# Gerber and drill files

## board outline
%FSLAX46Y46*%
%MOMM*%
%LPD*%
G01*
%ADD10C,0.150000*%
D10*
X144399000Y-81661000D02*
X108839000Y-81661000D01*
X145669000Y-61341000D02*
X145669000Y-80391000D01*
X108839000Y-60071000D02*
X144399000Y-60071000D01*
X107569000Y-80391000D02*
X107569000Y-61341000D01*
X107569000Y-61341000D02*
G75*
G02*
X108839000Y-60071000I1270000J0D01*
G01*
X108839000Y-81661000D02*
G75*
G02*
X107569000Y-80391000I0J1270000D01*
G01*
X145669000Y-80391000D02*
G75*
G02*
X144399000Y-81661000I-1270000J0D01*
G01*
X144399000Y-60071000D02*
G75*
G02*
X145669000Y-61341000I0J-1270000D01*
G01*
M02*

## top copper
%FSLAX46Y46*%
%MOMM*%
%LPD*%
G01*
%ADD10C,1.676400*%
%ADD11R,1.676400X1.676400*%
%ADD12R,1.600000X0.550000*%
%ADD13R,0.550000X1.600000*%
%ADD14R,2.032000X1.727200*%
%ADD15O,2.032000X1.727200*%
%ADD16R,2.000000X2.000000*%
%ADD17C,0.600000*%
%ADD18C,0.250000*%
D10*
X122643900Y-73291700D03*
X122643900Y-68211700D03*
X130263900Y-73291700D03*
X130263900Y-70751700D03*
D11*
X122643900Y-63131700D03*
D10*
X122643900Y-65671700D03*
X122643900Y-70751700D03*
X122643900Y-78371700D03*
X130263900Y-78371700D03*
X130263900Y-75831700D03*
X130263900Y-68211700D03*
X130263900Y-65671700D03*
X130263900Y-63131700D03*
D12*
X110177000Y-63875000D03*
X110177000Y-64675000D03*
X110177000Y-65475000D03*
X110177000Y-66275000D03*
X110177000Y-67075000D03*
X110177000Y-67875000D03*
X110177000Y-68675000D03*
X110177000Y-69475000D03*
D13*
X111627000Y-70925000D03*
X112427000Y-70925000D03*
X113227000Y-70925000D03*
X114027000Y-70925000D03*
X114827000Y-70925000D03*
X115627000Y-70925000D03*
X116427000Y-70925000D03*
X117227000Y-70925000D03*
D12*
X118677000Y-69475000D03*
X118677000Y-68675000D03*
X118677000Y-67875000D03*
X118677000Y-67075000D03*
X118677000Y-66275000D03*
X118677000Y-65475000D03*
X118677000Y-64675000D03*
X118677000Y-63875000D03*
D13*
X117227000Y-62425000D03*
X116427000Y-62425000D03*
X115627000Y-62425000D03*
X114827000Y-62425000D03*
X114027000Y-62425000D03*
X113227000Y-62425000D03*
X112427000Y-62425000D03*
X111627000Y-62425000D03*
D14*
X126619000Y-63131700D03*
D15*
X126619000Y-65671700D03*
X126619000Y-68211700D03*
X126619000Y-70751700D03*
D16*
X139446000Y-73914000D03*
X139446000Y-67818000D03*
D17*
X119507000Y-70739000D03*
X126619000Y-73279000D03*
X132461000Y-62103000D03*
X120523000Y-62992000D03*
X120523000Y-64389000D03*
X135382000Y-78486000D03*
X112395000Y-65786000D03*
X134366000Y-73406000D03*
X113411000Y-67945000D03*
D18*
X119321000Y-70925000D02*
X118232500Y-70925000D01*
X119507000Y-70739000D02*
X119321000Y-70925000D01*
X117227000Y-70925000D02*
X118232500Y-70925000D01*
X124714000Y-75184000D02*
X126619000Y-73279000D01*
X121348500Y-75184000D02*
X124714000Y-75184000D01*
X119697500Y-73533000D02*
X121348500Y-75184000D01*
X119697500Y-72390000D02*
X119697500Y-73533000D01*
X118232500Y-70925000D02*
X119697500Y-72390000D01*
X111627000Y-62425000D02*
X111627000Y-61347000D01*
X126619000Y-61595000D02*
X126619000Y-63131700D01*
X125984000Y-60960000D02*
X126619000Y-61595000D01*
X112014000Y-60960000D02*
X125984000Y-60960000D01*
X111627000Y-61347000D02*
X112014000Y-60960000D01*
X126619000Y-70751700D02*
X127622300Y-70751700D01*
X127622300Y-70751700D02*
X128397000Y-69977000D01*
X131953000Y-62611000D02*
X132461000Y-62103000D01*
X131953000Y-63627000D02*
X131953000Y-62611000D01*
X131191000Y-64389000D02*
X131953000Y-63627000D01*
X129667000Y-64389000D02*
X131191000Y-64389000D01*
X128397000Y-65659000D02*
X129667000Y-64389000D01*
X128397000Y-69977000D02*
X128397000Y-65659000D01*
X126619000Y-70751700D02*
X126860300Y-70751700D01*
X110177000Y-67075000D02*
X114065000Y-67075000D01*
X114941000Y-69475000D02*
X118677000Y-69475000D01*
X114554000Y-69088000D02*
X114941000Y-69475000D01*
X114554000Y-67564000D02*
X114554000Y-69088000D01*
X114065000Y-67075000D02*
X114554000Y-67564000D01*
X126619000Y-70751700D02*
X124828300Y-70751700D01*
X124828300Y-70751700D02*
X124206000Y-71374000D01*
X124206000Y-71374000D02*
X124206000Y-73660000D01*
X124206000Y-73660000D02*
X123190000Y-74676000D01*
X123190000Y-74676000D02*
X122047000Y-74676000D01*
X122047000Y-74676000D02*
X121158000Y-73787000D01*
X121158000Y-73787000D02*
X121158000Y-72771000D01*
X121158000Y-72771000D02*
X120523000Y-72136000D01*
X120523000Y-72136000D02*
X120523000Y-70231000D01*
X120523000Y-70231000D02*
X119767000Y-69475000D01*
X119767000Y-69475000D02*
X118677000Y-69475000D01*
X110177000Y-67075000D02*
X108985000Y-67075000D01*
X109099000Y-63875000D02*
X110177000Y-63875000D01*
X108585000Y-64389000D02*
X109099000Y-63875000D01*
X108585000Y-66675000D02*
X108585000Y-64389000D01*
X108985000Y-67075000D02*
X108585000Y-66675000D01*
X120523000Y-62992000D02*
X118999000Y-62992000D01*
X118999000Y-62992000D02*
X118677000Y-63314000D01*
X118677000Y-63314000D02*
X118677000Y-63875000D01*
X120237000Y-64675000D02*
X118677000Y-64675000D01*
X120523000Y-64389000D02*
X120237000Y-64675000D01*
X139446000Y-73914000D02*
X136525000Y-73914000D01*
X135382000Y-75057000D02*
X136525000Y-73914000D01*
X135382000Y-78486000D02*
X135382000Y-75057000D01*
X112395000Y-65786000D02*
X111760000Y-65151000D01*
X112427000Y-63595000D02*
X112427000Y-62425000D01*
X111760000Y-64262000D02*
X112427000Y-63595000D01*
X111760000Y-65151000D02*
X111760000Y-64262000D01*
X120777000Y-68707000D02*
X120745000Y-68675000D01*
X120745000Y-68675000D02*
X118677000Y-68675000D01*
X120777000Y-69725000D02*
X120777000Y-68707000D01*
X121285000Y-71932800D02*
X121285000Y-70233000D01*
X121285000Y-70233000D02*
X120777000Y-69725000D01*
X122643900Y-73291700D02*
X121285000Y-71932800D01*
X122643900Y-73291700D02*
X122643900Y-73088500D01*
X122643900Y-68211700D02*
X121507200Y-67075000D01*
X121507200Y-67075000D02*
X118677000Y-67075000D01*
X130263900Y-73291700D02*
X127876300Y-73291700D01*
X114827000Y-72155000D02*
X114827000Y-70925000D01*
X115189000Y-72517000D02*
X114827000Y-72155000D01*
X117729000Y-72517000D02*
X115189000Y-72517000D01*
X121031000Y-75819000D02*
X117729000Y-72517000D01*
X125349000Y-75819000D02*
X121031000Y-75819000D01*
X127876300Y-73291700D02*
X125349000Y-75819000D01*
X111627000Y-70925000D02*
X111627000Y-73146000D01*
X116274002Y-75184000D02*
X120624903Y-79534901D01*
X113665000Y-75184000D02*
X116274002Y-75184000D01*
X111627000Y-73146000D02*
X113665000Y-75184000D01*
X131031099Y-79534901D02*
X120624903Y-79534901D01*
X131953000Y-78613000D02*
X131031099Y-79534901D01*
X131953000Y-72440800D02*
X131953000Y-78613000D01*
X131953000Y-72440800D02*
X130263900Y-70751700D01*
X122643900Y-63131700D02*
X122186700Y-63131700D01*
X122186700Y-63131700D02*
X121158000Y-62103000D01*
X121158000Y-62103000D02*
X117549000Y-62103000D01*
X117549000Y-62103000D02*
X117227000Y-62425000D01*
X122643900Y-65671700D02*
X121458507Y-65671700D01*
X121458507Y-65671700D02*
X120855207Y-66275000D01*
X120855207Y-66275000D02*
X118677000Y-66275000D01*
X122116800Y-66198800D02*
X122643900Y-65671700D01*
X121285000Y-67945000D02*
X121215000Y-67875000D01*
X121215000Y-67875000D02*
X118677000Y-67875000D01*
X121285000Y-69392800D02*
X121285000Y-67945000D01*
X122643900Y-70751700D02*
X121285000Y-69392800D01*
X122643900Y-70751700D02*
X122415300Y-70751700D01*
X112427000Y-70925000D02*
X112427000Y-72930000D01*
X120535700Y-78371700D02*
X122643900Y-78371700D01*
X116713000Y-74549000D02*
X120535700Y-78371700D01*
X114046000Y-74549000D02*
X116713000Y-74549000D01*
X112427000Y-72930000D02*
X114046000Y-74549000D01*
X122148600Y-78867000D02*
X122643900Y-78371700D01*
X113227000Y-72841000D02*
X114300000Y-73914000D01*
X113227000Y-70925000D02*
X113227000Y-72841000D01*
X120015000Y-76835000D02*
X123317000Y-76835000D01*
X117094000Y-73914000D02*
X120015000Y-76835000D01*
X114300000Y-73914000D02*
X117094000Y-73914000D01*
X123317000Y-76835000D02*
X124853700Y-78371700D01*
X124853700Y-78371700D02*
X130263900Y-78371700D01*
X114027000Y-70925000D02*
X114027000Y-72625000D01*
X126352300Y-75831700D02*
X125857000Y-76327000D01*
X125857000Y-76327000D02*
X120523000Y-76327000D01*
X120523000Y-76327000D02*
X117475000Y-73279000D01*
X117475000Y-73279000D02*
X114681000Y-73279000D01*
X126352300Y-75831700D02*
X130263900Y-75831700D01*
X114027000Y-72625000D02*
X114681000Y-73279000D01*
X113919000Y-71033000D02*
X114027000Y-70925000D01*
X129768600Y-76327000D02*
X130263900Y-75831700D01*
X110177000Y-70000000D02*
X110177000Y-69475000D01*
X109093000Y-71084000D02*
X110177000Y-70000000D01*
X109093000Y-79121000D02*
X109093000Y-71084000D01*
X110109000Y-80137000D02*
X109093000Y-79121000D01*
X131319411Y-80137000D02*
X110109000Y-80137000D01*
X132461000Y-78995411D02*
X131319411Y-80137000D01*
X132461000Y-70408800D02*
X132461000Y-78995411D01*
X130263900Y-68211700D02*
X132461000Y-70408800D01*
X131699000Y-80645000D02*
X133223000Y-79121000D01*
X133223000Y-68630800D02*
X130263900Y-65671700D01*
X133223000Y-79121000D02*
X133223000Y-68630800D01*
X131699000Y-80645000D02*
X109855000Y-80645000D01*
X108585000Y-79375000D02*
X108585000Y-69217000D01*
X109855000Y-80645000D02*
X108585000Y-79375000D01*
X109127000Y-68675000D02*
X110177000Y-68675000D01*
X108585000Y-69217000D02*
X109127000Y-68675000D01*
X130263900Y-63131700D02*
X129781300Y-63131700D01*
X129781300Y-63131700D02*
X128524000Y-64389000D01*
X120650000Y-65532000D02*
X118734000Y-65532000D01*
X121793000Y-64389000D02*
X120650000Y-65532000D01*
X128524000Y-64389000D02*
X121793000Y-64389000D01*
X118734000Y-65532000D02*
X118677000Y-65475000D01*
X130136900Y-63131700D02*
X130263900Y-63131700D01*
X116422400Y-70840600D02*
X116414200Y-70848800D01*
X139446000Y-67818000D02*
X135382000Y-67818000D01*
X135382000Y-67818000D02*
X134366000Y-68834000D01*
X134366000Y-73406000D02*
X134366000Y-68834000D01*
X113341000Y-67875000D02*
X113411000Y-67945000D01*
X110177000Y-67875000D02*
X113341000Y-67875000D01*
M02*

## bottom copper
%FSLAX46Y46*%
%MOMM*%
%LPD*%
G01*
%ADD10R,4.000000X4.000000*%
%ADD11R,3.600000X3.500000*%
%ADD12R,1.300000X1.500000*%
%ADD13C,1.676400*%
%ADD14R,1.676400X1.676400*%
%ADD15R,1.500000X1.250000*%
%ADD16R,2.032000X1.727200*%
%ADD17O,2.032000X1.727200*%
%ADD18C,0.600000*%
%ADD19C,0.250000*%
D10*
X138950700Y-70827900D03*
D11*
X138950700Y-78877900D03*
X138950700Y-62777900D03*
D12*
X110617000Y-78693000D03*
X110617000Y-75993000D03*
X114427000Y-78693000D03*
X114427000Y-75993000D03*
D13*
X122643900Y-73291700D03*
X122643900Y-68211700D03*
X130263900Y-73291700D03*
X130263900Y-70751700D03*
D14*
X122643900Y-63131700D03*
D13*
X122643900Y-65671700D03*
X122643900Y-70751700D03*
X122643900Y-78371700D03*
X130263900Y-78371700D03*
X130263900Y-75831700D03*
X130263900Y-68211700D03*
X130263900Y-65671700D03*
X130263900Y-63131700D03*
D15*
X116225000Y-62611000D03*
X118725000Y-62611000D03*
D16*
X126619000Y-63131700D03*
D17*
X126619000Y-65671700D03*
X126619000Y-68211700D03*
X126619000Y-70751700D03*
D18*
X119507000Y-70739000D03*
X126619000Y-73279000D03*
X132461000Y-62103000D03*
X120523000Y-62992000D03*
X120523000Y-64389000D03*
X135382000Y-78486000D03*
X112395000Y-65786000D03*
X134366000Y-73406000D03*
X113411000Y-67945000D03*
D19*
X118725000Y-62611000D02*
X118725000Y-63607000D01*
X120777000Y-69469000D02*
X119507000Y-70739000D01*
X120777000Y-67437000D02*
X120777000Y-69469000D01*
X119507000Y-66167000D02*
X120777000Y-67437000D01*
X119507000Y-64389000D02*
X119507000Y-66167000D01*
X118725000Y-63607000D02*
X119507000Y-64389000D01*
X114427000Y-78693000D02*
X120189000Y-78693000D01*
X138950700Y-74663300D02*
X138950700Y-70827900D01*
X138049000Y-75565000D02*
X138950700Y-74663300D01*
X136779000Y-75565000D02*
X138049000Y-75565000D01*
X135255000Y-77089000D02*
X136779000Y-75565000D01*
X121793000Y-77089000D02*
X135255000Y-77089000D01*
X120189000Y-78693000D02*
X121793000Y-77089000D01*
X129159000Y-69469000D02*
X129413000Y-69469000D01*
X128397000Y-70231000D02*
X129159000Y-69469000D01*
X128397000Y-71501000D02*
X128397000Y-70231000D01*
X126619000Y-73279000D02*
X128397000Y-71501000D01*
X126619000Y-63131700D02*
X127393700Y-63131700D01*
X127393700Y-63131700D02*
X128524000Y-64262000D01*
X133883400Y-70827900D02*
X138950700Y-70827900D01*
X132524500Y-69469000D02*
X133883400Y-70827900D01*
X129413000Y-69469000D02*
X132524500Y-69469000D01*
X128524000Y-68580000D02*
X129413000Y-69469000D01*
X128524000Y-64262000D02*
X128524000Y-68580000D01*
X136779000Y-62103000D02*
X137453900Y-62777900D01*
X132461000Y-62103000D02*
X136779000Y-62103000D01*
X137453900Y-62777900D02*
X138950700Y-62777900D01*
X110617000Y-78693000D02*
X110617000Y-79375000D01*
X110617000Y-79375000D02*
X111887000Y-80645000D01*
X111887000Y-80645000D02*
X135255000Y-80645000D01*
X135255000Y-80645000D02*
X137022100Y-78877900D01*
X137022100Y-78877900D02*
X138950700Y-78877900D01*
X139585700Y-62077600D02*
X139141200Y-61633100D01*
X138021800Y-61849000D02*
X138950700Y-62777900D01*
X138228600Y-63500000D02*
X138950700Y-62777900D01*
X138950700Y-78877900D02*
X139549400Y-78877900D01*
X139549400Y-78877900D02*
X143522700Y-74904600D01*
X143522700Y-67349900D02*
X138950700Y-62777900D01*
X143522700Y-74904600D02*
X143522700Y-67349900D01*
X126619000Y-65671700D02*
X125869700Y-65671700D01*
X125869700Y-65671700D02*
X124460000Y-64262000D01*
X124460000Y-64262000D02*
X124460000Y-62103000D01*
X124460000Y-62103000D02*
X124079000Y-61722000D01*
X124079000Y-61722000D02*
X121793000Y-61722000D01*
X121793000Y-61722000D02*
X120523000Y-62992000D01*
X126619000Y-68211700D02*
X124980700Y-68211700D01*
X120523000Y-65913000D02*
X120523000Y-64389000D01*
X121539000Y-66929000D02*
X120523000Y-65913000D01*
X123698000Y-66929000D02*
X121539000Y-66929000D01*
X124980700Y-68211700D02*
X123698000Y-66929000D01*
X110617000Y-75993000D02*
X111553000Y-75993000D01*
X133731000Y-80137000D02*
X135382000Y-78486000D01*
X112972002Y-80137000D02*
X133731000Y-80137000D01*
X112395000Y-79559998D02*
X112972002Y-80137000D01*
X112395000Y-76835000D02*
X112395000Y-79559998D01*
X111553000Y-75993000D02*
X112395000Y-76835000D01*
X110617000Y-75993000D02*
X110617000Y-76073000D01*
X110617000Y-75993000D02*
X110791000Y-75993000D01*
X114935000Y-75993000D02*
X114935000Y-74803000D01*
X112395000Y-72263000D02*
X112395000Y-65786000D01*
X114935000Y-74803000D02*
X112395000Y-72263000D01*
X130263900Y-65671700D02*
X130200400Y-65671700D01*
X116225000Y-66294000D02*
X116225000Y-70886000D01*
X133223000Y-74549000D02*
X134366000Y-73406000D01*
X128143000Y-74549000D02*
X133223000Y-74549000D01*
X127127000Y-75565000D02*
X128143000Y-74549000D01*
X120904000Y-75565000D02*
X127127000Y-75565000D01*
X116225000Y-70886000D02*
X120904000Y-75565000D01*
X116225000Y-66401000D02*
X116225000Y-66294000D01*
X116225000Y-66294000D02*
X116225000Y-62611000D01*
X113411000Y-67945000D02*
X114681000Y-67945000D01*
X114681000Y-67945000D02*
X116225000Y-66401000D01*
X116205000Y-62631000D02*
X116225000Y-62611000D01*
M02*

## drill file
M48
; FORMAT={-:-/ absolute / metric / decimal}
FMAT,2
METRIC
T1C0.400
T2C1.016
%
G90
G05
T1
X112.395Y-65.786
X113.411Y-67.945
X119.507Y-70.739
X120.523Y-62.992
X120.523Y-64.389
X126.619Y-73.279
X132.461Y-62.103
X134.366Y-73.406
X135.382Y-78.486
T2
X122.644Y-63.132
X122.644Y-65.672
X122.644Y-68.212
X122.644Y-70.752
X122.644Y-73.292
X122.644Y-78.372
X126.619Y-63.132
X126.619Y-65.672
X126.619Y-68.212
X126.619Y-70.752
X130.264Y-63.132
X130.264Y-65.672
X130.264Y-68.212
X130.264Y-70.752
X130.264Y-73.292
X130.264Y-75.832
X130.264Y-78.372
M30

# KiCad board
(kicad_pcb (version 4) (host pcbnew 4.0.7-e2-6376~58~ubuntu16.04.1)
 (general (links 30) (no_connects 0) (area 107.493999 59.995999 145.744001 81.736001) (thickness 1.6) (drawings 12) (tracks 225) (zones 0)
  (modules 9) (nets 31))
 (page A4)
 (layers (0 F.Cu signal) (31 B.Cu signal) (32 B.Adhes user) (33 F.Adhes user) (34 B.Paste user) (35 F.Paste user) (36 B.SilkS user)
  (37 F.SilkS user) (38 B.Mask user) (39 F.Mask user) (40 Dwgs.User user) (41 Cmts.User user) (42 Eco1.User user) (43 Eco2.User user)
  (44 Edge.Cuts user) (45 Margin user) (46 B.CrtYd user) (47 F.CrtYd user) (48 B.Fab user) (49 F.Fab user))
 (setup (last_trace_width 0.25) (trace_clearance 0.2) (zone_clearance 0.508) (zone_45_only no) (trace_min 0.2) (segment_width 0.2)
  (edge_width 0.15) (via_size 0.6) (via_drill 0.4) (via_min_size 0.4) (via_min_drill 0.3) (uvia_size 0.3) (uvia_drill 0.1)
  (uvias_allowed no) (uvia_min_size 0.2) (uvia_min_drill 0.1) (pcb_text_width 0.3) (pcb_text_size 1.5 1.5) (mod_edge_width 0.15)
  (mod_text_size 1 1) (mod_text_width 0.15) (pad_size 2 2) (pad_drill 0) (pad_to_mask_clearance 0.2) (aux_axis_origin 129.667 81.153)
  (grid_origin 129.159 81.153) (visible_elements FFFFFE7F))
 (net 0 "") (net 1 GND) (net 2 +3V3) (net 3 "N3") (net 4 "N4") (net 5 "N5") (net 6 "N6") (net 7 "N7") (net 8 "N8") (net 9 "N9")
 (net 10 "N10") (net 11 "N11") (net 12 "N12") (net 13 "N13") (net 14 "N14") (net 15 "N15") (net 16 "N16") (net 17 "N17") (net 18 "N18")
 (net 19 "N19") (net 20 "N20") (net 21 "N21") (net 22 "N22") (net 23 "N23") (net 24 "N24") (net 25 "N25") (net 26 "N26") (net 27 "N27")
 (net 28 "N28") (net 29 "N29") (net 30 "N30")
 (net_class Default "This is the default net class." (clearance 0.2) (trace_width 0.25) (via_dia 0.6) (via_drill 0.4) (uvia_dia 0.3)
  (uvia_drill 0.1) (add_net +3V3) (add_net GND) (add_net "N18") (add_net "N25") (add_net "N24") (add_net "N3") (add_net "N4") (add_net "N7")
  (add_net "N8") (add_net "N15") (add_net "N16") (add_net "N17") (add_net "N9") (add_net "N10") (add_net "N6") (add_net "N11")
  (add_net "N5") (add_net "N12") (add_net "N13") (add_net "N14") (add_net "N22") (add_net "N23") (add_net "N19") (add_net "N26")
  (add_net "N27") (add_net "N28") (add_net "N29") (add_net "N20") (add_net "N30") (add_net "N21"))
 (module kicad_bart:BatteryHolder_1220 (layer B.Cu) (at 138.9507 70.8279 270)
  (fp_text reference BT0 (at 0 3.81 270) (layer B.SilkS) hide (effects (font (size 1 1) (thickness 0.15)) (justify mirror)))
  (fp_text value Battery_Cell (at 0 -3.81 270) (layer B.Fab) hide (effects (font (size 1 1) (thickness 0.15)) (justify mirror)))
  (pad 2 smd rect (at 0 0 270) (size 4 4) (layers B.Cu B.Paste B.Mask) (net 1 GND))
  (pad 1 smd rect (at 8.05 0 270) (size 3.5 3.6) (layers B.Cu B.Paste B.Mask) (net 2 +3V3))
  (pad 1 smd rect (at -8.05 0 270) (size 3.5 3.6) (layers B.Cu B.Paste B.Mask) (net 2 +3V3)))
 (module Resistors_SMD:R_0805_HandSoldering (layer B.Cu) (at 110.617 77.343 90)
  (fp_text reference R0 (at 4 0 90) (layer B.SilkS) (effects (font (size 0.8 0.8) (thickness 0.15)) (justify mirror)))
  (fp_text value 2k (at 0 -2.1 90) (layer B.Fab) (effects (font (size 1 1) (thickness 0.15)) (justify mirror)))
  (pad 1 smd rect (at -1.35 0 90) (size 1.5 1.3) (layers B.Cu B.Paste B.Mask) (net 2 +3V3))
  (pad 2 smd rect (at 1.35 0 90) (size 1.5 1.3) (layers B.Cu B.Paste B.Mask) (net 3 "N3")))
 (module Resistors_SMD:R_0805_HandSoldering (layer B.Cu) (at 114.427 77.343 90)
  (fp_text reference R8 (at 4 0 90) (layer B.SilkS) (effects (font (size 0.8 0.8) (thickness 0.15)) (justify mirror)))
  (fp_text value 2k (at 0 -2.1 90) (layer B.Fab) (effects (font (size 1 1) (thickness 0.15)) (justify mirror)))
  (pad 1 smd rect (at -1.35 0 90) (size 1.5 1.3) (layers B.Cu B.Paste B.Mask) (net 1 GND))
  (pad 2 smd rect (at 1.35 0 90) (size 1.5 1.3) (layers B.Cu B.Paste B.Mask) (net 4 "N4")))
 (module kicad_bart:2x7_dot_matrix (layer F.Cu) (at 126.4539 70.7517 270)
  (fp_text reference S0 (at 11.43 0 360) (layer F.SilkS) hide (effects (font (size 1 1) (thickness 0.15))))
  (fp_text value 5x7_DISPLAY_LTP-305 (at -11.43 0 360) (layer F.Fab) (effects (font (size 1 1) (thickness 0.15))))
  (pad 5C thru_hole circle (at 2.54 3.81 270) (size 1.6764 1.6764) (drill 1.016) (layers *.Cu *.Mask F.SilkS) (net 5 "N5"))
  (pad 3 thru_hole circle (at -2.54 3.81 270) (size 1.6764 1.6764) (drill 1.016) (layers *.Cu *.Mask F.SilkS) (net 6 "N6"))
  (pad 10 thru_hole circle (at 2.54 -3.81 270) (size 1.6764 1.6764) (drill 1.016) (layers *.Cu *.Mask F.SilkS) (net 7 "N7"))
  (pad 11 thru_hole circle (at 0 -3.81 270) (size 1.6764 1.6764) (drill 1.016) (layers *.Cu *.Mask F.SilkS) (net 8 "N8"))
  (pad 1C thru_hole rect (at -7.62 3.81 270) (size 1.6764 1.6764) (drill 1.016) (layers *.Cu *.Mask F.SilkS) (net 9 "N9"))
  (pad 2 thru_hole circle (at -5.08 3.81 270) (size 1.6764 1.6764) (drill 1.016) (layers *.Cu *.Mask F.SilkS) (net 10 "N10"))
  (pad 4 thru_hole circle (at 0 3.81 270) (size 1.6764 1.6764) (drill 1.016) (layers *.Cu *.Mask F.SilkS) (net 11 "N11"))
  (pad 7 thru_hole circle (at 7.62 3.81 270) (size 1.6764 1.6764) (drill 1.016) (layers *.Cu *.Mask F.SilkS) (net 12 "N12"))
  (pad 8C thru_hole circle (at 7.62 -3.81 270) (size 1.6764 1.6764) (drill 1.016) (layers *.Cu *.Mask F.SilkS) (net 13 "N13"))
  (pad 9 thru_hole circle (at 5.08 -3.81 270) (size 1.6764 1.6764) (drill 1.016) (layers *.Cu *.Mask F.SilkS) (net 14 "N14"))
  (pad 12 thru_hole circle (at -2.54 -3.81 270) (size 1.6764 1.6764) (drill 1.016) (layers *.Cu *.Mask F.SilkS) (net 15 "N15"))
  (pad 13C thru_hole circle (at -5.08 -3.81 270) (size 1.6764 1.6764) (drill 1.016) (layers *.Cu *.Mask F.SilkS) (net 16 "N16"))
  (pad 14C thru_hole circle (at -7.62 -3.81 270) (size 1.6764 1.6764) (drill 1.016) (layers *.Cu *.Mask F.SilkS) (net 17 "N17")))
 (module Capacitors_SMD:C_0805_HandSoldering (layer B.Cu) (at 117.475 62.611)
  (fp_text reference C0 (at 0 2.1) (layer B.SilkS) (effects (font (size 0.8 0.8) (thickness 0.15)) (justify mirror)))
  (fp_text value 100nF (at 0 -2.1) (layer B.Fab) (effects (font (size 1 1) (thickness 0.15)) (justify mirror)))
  (pad 1 smd rect (at -1.25 0) (size 1.5 1.25) (layers B.Cu B.Paste B.Mask) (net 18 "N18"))
  (pad 2 smd rect (at 1.25 0) (size 1.5 1.25) (layers B.Cu B.Paste B.Mask) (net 1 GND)))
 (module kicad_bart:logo (layer F.Cu) (at 140.843 77.851)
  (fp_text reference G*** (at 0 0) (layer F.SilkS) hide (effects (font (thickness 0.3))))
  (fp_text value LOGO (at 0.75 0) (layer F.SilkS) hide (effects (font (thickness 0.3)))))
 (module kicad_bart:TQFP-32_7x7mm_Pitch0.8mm (layer F.Cu) (at 114.427 66.675)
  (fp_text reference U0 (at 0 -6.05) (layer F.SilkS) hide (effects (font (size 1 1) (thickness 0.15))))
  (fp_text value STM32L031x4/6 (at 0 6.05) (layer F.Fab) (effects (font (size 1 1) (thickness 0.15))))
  (pad 1 smd rect (at -4.25 -2.8) (size 1.6 0.55) (layers F.Cu F.Paste F.Mask) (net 2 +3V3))
  (pad 2 smd rect (at -4.25 -2) (size 1.6 0.55) (layers F.Cu F.Paste F.Mask) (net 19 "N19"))
  (pad 3 smd rect (at -4.25 -1.2) (size 1.6 0.55) (layers F.Cu F.Paste F.Mask) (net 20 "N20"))
  (pad 4 smd rect (at -4.25 -0.4) (size 1.6 0.55) (layers F.Cu F.Paste F.Mask) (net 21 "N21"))
  (pad 5 smd rect (at -4.25 0.4) (size 1.6 0.55) (layers F.Cu F.Paste F.Mask) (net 2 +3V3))
  (pad 6 smd rect (at -4.25 1.2) (size 1.6 0.55) (layers F.Cu F.Paste F.Mask) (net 18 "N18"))
  (pad 7 smd rect (at -4.25 2) (size 1.6 0.55) (layers F.Cu F.Paste F.Mask) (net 16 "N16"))
  (pad 8 smd rect (at -4.25 2.8) (size 1.6 0.55) (layers F.Cu F.Paste F.Mask) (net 15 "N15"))
  (pad 9 smd rect (at -2.8 4.25 90) (size 1.6 0.55) (layers F.Cu F.Paste F.Mask) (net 8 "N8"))
  (pad 10 smd rect (at -2 4.25 90) (size 1.6 0.55) (layers F.Cu F.Paste F.Mask) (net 12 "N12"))
  (pad 11 smd rect (at -1.2 4.25 90) (size 1.6 0.55) (layers F.Cu F.Paste F.Mask) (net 13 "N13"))
  (pad 12 smd rect (at -0.4 4.25 90) (size 1.6 0.55) (layers F.Cu F.Paste F.Mask) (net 14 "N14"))
  (pad 13 smd rect (at 0.4 4.25 90) (size 1.6 0.55) (layers F.Cu F.Paste F.Mask) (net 7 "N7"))
  (pad 14 smd rect (at 1.2 4.25 90) (size 1.6 0.55) (layers F.Cu F.Paste F.Mask) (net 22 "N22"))
  (pad 15 smd rect (at 2 4.25 90) (size 1.6 0.55) (layers F.Cu F.Paste F.Mask) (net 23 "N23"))
  (pad 16 smd rect (at 2.8 4.25 90) (size 1.6 0.55) (layers F.Cu F.Paste F.Mask) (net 1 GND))
  (pad 17 smd rect (at 4.25 2.8) (size 1.6 0.55) (layers F.Cu F.Paste F.Mask) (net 2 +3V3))
  (pad 18 smd rect (at 4.25 2) (size 1.6 0.55) (layers F.Cu F.Paste F.Mask) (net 5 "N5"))
  (pad 19 smd rect (at 4.25 1.2) (size 1.6 0.55) (layers F.Cu F.Paste F.Mask) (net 11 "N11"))
  (pad 20 smd rect (at 4.25 0.4) (size 1.6 0.55) (layers F.Cu F.Paste F.Mask) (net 6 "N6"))
  (pad 21 smd rect (at 4.25 -0.4) (size 1.6 0.55) (layers F.Cu F.Paste F.Mask) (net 10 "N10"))
  (pad 22 smd rect (at 4.25 -1.2) (size 1.6 0.55) (layers F.Cu F.Paste F.Mask) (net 17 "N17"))
  (pad 23 smd rect (at 4.25 -2) (size 1.6 0.55) (layers F.Cu F.Paste F.Mask) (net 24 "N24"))
  (pad 24 smd rect (at 4.25 -2.8) (size 1.6 0.55) (layers F.Cu F.Paste F.Mask) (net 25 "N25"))
  (pad 25 smd rect (at 2.8 -4.25 90) (size 1.6 0.55) (layers F.Cu F.Paste F.Mask) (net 9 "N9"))
  (pad 26 smd rect (at 2 -4.25 90) (size 1.6 0.55) (layers F.Cu F.Paste F.Mask) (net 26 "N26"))
  (pad 27 smd rect (at 1.2 -4.25 90) (size 1.6 0.55) (layers F.Cu F.Paste F.Mask) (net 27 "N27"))
  (pad 28 smd rect (at 0.4 -4.25 90) (size 1.6 0.55) (layers F.Cu F.Paste F.Mask) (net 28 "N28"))
  (pad 29 smd rect (at -0.4 -4.25 90) (size 1.6 0.55) (layers F.Cu F.Paste F.Mask) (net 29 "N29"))
  (pad 30 smd rect (at -1.2 -4.25 90) (size 1.6 0.55) (layers F.Cu F.Paste F.Mask) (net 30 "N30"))
  (pad 31 smd rect (at -2 -4.25 90) (size 1.6 0.55) (layers F.Cu F.Paste F.Mask) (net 4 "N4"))
  (pad 32 smd rect (at -2.8 -4.25 90) (size 1.6 0.55) (layers F.Cu F.Paste F.Mask) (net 1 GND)))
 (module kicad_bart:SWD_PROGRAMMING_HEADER (layer F.Cu) (at 126.619 63.1317)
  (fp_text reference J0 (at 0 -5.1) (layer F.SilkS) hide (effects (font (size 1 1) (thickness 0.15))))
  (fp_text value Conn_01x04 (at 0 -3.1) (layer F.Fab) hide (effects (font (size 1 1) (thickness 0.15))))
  (pad 1 thru_hole rect (at 0 0) (size 2.032 1.7272) (drill 1.016) (layers *.Cu *.Mask F.SilkS) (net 1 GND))
  (pad 2 thru_hole oval (at 0 2.54) (size 2.032 1.7272) (drill 1.016) (layers *.Cu *.Mask F.SilkS) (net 25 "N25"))
  (pad 3 thru_hole oval (at 0 5.08) (size 2.032 1.7272) (drill 1.016) (layers *.Cu *.Mask F.SilkS) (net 24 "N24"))
  (pad 4 thru_hole oval (at 0 7.62) (size 2.032 1.7272) (drill 1.016) (layers *.Cu *.Mask F.SilkS) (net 2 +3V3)))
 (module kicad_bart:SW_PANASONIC (layer F.Cu) (at 139.446 70.866 270)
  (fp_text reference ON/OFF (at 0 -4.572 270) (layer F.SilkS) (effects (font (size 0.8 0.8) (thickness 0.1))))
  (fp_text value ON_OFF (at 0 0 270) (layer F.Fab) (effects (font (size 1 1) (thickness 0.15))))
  (pad 2 smd rect (at 3.048 0 270) (size 2 2) (layers F.Cu F.Paste F.Mask) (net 3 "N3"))
  (pad 1 smd rect (at -3.048 0 270) (size 2 2) (layers F.Cu F.Paste F.Mask) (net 18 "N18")))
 (gr_line (start 144.399 81.661) (end 108.839 81.661) (angle 90) (layer Edge.Cuts) (width 0.15))
 (gr_line (start 145.669 61.341) (end 145.669 80.391) (angle 90) (layer Edge.Cuts) (width 0.15))
 (gr_line (start 108.839 60.071) (end 144.399 60.071) (angle 90) (layer Edge.Cuts) (width 0.15))
 (gr_line (start 107.569 80.391) (end 107.569 61.341) (angle 90) (layer Edge.Cuts) (width 0.15))
 (gr_arc (start 108.839 61.341) (end 107.569 61.341) (angle 90) (layer Edge.Cuts) (width 0.15))
 (gr_arc (start 108.839 80.391) (end 108.839 81.661) (angle 90) (layer Edge.Cuts) (width 0.15))
 (gr_arc (start 144.399 80.391) (end 145.669 80.391) (angle 90) (layer Edge.Cuts) (width 0.15))
 (gr_arc (start 144.399 61.341) (end 144.399 60.071) (angle 90) (layer Edge.Cuts) (width 0.15))
 (segment (start 118.725 62.611) (end 118.725 63.607) (width 0.25) (layer B.Cu) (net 1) (status 10))
 (segment (start 119.321 70.925) (end 118.2325 70.925) (width 0.25) (layer F.Cu) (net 1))
 (segment (start 119.507 70.739) (end 119.321 70.925) (width 0.25) (layer F.Cu) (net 1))
 (via (at 119.507 70.739) (size 0.6) (drill 0.4) (layers F.Cu B.Cu) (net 1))
 (segment (start 120.777 69.469) (end 119.507 70.739) (width 0.25) (layer B.Cu) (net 1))
 (segment (start 120.777 67.437) (end 120.777 69.469) (width 0.25) (layer B.Cu) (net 1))
 (segment (start 119.507 66.167) (end 120.777 67.437) (width 0.25) (layer B.Cu) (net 1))
 (segment (start 119.507 64.389) (end 119.507 66.167) (width 0.25) (layer B.Cu) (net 1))
 (segment (start 118.725 63.607) (end 119.507 64.389) (width 0.25) (layer B.Cu) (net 1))
 (segment (start 114.427 78.693) (end 120.189 78.693) (width 0.25) (layer B.Cu) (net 1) (status 10))
 (segment (start 138.9507 74.6633) (end 138.9507 70.8279) (width 0.25) (layer B.Cu) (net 1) (status 20))
 (segment (start 138.049 75.565) (end 138.9507 74.6633) (width 0.25) (layer B.Cu) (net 1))
 (segment (start 136.779 75.565) (end 138.049 75.565) (width 0.25) (layer B.Cu) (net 1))
 (segment (start 135.255 77.089) (end 136.779 75.565) (width 0.25) (layer B.Cu) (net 1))
 (segment (start 121.793 77.089) (end 135.255 77.089) (width 0.25) (layer B.Cu) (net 1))
 (segment (start 120.189 78.693) (end 121.793 77.089) (width 0.25) (layer B.Cu) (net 1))
 (segment (start 117.227 70.925) (end 118.2325 70.925) (width 0.25) (layer F.Cu) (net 1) (status 10))
 (segment (start 129.159 69.469) (end 129.413 69.469) (width 0.25) (layer B.Cu) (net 1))
 (segment (start 128.397 70.231) (end 129.159 69.469) (width 0.25) (layer B.Cu) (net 1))
 (segment (start 128.397 71.501) (end 128.397 70.231) (width 0.25) (layer B.Cu) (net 1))
 (segment (start 126.619 73.279) (end 128.397 71.501) (width 0.25) (layer B.Cu) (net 1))
 (via (at 126.619 73.279) (size 0.6) (drill 0.4) (layers F.Cu B.Cu) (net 1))
 (segment (start 124.714 75.184) (end 126.619 73.279) (width 0.25) (layer F.Cu) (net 1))
 (segment (start 121.3485 75.184) (end 124.714 75.184) (width 0.25) (layer F.Cu) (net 1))
 (segment (start 119.6975 73.533) (end 121.3485 75.184) (width 0.25) (layer F.Cu) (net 1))
 (segment (start 119.6975 72.39) (end 119.6975 73.533) (width 0.25) (layer F.Cu) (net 1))
 (segment (start 118.2325 70.925) (end 119.6975 72.39) (width 0.25) (layer F.Cu) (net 1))
 (segment (start 126.619 63.1317) (end 127.3937 63.1317) (width 0.25) (layer B.Cu) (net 1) (status 30))
 (segment (start 127.3937 63.1317) (end 128.524 64.262) (width 0.25) (layer B.Cu) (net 1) (status 10))
 (segment (start 133.8834 70.8279) (end 138.9507 70.8279) (width 0.25) (layer B.Cu) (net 1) (status 20))
 (segment (start 132.5245 69.469) (end 133.8834 70.8279) (width 0.25) (layer B.Cu) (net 1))
 (segment (start 129.413 69.469) (end 132.5245 69.469) (width 0.25) (layer B.Cu) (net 1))
 (segment (start 128.524 68.58) (end 129.413 69.469) (width 0.25) (layer B.Cu) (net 1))
 (segment (start 128.524 64.262) (end 128.524 68.58) (width 0.25) (layer B.Cu) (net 1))
 (segment (start 111.627 62.425) (end 111.627 61.347) (width 0.25) (layer F.Cu) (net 1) (status 10))
 (segment (start 126.619 61.595) (end 126.619 63.1317) (width 0.25) (layer F.Cu) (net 1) (status 20))
 (segment (start 125.984 60.96) (end 126.619 61.595) (width 0.25) (layer F.Cu) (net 1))
 (segment (start 112.014 60.96) (end 125.984 60.96) (width 0.25) (layer F.Cu) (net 1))
 (segment (start 111.627 61.347) (end 112.014 60.96) (width 0.25) (layer F.Cu) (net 1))
 (segment (start 126.619 70.7517) (end 127.6223 70.7517) (width 0.25) (layer F.Cu) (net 2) (status 30))
 (segment (start 127.6223 70.7517) (end 128.397 69.977) (width 0.25) (layer F.Cu) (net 2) (status 10))
 (segment (start 136.779 62.103) (end 137.4539 62.7779) (width 0.25) (layer B.Cu) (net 2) (status 20))
 (segment (start 132.461 62.103) (end 136.779 62.103) (width 0.25) (layer B.Cu) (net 2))
 (via (at 132.461 62.103) (size 0.6) (drill 0.4) (layers F.Cu B.Cu) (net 2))
 (segment (start 131.953 62.611) (end 132.461 62.103) (width 0.25) (layer F.Cu) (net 2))
 (segment (start 131.953 63.627) (end 131.953 62.611) (width 0.25) (layer F.Cu) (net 2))
 (segment (start 131.191 64.389) (end 131.953 63.627) (width 0.25) (layer F.Cu) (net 2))
 (segment (start 129.667 64.389) (end 131.191 64.389) (width 0.25) (layer F.Cu) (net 2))
 (segment (start 128.397 65.659) (end 129.667 64.389) (width 0.25) (layer F.Cu) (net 2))
 (segment (start 128.397 69.977) (end 128.397 65.659) (width 0.25) (layer F.Cu) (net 2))
 (segment (start 137.4539 62.7779) (end 138.9507 62.7779) (width 0.25) (layer B.Cu) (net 2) (status 30))
 (segment (start 110.617 78.693) (end 110.617 79.375) (width 0.25) (layer B.Cu) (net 2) (status 30))
 (segment (start 110.617 79.375) (end 111.887 80.645) (width 0.25) (layer B.Cu) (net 2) (status 10))
 (segment (start 111.887 80.645) (end 135.255 80.645) (width 0.25) (layer B.Cu) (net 2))
 (segment (start 135.255 80.645) (end 137.0221 78.8779) (width 0.25) (layer B.Cu) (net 2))
 (segment (start 137.0221 78.8779) (end 138.9507 78.8779) (width 0.25) (layer B.Cu) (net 2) (status 20))
 (segment (start 126.619 70.7517) (end 126.8603 70.7517) (width 0.25) (layer F.Cu) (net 2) (status 30))
 (segment (start 110.177 67.075) (end 114.065 67.075) (width 0.25) (layer F.Cu) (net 2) (status 10))
 (segment (start 114.941 69.475) (end 118.677 69.475) (width 0.25) (layer F.Cu) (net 2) (status 20))
 (segment (start 114.554 69.088) (end 114.941 69.475) (width 0.25) (layer F.Cu) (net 2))
 (segment (start 114.554 67.564) (end 114.554 69.088) (width 0.25) (layer F.Cu) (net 2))
 (segment (start 114.065 67.075) (end 114.554 67.564) (width 0.25) (layer F.Cu) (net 2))
 (segment (start 126.619 70.7517) (end 124.8283 70.7517) (width 0.25) (layer F.Cu) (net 2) (status 10))
 (segment (start 124.8283 70.7517) (end 124.206 71.374) (width 0.25) (layer F.Cu) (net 2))
 (segment (start 124.206 71.374) (end 124.206 73.66) (width 0.25) (layer F.Cu) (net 2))
 (segment (start 124.206 73.66) (end 123.19 74.676) (width 0.25) (layer F.Cu) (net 2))
 (segment (start 123.19 74.676) (end 122.047 74.676) (width 0.25) (layer F.Cu) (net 2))
 (segment (start 122.047 74.676) (end 121.158 73.787) (width 0.25) (layer F.Cu) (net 2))
 (segment (start 121.158 73.787) (end 121.158 72.771) (width 0.25) (layer F.Cu) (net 2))
 (segment (start 121.158 72.771) (end 120.523 72.136) (width 0.25) (layer F.Cu) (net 2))
 (segment (start 120.523 72.136) (end 120.523 70.231) (width 0.25) (layer F.Cu) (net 2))
 (segment (start 120.523 70.231) (end 119.767 69.475) (width 0.25) (layer F.Cu) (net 2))
 (segment (start 119.767 69.475) (end 118.677 69.475) (width 0.25) (layer F.Cu) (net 2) (status 20))
 (segment (start 110.177 67.075) (end 108.985 67.075) (width 0.25) (layer F.Cu) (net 2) (status 10))
 (segment (start 109.099 63.875) (end 110.177 63.875) (width 0.25) (layer F.Cu) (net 2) (status 20))
 (segment (start 108.585 64.389) (end 109.099 63.875) (width 0.25) (layer F.Cu) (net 2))
 (segment (start 108.585 66.675) (end 108.585 64.389) (width 0.25) (layer F.Cu) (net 2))
 (segment (start 108.985 67.075) (end 108.585 66.675) (width 0.25) (layer F.Cu) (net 2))
 (segment (start 139.5857 62.0776) (end 139.1412 61.6331) (width 0.25) (layer B.Cu) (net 2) (status 30))
 (segment (start 138.0218 61.849) (end 138.9507 62.7779) (width 0.25) (layer B.Cu) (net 2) (status 30))
 (segment (start 138.2286 63.5) (end 138.9507 62.7779) (width 0.25) (layer B.Cu) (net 2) (status 30))
 (segment (start 138.9507 78.8779) (end 139.5494 78.8779) (width 0.25) (layer B.Cu) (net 2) (status 30))
 (segment (start 139.5494 78.8779) (end 143.5227 74.9046) (width 0.25) (layer B.Cu) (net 2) (status 10))
 (segment (start 143.5227 67.3499) (end 138.9507 62.7779) (width 0.25) (layer B.Cu) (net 2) (status 20))
 (segment (start 143.5227 74.9046) (end 143.5227 67.3499) (width 0.25) (layer B.Cu) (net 2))
 (segment (start 126.619 65.6717) (end 125.8697 65.6717) (width 0.25) (layer B.Cu) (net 25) (status 30))
 (segment (start 125.8697 65.6717) (end 124.46 64.262) (width 0.25) (layer B.Cu) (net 25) (status 10))
 (segment (start 124.46 64.262) (end 124.46 62.103) (width 0.25) (layer B.Cu) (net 25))
 (segment (start 124.46 62.103) (end 124.079 61.722) (width 0.25) (layer B.Cu) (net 25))
 (segment (start 124.079 61.722) (end 121.793 61.722) (width 0.25) (layer B.Cu) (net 25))
 (segment (start 121.793 61.722) (end 120.523 62.992) (width 0.25) (layer B.Cu) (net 25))
 (via (at 120.523 62.992) (size 0.6) (drill 0.4) (layers F.Cu B.Cu) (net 25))
 (segment (start 120.523 62.992) (end 118.999 62.992) (width 0.25) (layer F.Cu) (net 25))
 (segment (start 118.999 62.992) (end 118.677 63.314) (width 0.25) (layer F.Cu) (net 25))
 (segment (start 118.677 63.314) (end 118.677 63.875) (width 0.25) (layer F.Cu) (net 25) (status 20))
 (segment (start 126.619 68.2117) (end 124.9807 68.2117) (width 0.25) (layer B.Cu) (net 24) (status 10))
 (segment (start 120.237 64.675) (end 118.677 64.675) (width 0.25) (layer F.Cu) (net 24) (status 20))
 (segment (start 120.523 64.389) (end 120.237 64.675) (width 0.25) (layer F.Cu) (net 24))
 (via (at 120.523 64.389) (size 0.6) (drill 0.4) (layers F.Cu B.Cu) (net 24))
 (segment (start 120.523 65.913) (end 120.523 64.389) (width 0.25) (layer B.Cu) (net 24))
 (segment (start 121.539 66.929) (end 120.523 65.913) (width 0.25) (layer B.Cu) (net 24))
 (segment (start 123.698 66.929) (end 121.539 66.929) (width 0.25) (layer B.Cu) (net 24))
 (segment (start 124.9807 68.2117) (end 123.698 66.929) (width 0.25) (layer B.Cu) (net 24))
 (segment (start 139.446 73.914) (end 136.525 73.914) (width 0.25) (layer F.Cu) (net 3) (status 10))
 (segment (start 110.617 75.993) (end 111.553 75.993) (width 0.25) (layer B.Cu) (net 3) (status 10))
 (segment (start 135.382 75.057) (end 136.525 73.914) (width 0.25) (layer F.Cu) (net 3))
 (segment (start 135.382 78.486) (end 135.382 75.057) (width 0.25) (layer F.Cu) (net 3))
 (via (at 135.382 78.486) (size 0.6) (drill 0.4) (layers F.Cu B.Cu) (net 3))
 (segment (start 133.731 80.137) (end 135.382 78.486) (width 0.25) (layer B.Cu) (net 3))
 (segment (start 112.972002 80.137) (end 133.731 80.137) (width 0.25) (layer B.Cu) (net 3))
 (segment (start 112.395 79.559998) (end 112.972002 80.137) (width 0.25) (layer B.Cu) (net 3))
 (segment (start 112.395 76.835) (end 112.395 79.559998) (width 0.25) (layer B.Cu) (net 3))
 (segment (start 111.553 75.993) (end 112.395 76.835) (width 0.25) (layer B.Cu) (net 3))
 (segment (start 110.617 75.993) (end 110.617 76.073) (width 0.25) (layer B.Cu) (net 3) (status 30))
 (segment (start 110.617 75.993) (end 110.791 75.993) (width 0.25) (layer B.Cu) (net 3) (status 30))
 (segment (start 112.395 65.786) (end 111.76 65.151) (width 0.25) (layer F.Cu) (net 4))
 (segment (start 112.427 63.595) (end 112.427 62.425) (width 0.25) (layer F.Cu) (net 4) (status 20))
 (segment (start 111.76 64.262) (end 112.427 63.595) (width 0.25) (layer F.Cu) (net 4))
 (segment (start 111.76 65.151) (end 111.76 64.262) (width 0.25) (layer F.Cu) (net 4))
 (segment (start 114.935 75.993) (end 114.935 74.803) (width 0.25) (layer B.Cu) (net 4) (status 10))
 (via (at 112.395 65.786) (size 0.6) (drill 0.4) (layers F.Cu B.Cu) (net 4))
 (segment (start 112.395 72.263) (end 112.395 65.786) (width 0.25) (layer B.Cu) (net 4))
 (segment (start 114.935 74.803) (end 112.395 72.263) (width 0.25) (layer B.Cu) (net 4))
 (segment (start 120.777 68.707) (end 120.745 68.675) (width 0.25) (layer F.Cu) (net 5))
 (segment (start 120.745 68.675) (end 118.677 68.675) (width 0.25) (layer F.Cu) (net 5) (status 20))
 (segment (start 120.777 69.725) (end 120.777 68.707) (width 0.25) (layer F.Cu) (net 5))
 (segment (start 121.285 71.9328) (end 121.285 70.233) (width 0.25) (layer F.Cu) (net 5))
 (segment (start 121.285 70.233) (end 120.777 69.725) (width 0.25) (layer F.Cu) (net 5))
 (segment (start 122.6439 73.2917) (end 121.285 71.9328) (width 0.25) (layer F.Cu) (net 5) (status 10))
 (segment (start 122.6439 73.2917) (end 122.6439 73.0885) (width 0.25) (layer F.Cu) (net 5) (status 30))
 (segment (start 122.6439 68.2117) (end 121.5072 67.075) (width 0.25) (layer F.Cu) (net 6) (status 10))
 (segment (start 121.5072 67.075) (end 118.677 67.075) (width 0.25) (layer F.Cu) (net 6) (status 20))
 (segment (start 130.2639 73.2917) (end 127.8763 73.2917) (width 0.25) (layer F.Cu) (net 7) (status 10))
 (segment (start 114.827 72.155) (end 114.827 70.925) (width 0.25) (layer F.Cu) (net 7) (status 20))
 (segment (start 115.189 72.517) (end 114.827 72.155) (width 0.25) (layer F.Cu) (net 7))
 (segment (start 117.729 72.517) (end 115.189 72.517) (width 0.25) (layer F.Cu) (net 7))
 (segment (start 121.031 75.819) (end 117.729 72.517) (width 0.25) (layer F.Cu) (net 7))
 (segment (start 125.349 75.819) (end 121.031 75.819) (width 0.25) (layer F.Cu) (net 7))
 (segment (start 127.8763 73.2917) (end 125.349 75.819) (width 0.25) (layer F.Cu) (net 7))
 (segment (start 111.627 70.925) (end 111.627 73.146) (width 0.25) (layer F.Cu) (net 8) (status 10))
 (segment (start 116.274002 75.184) (end 120.624903 79.534901) (width 0.25) (layer F.Cu) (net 8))
 (segment (start 113.665 75.184) (end 116.274002 75.184) (width 0.25) (layer F.Cu) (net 8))
 (segment (start 111.627 73.146) (end 113.665 75.184) (width 0.25) (layer F.Cu) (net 8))
 (segment (start 131.031099 79.534901) (end 120.624903 79.534901) (width 0.25) (layer F.Cu) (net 8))
 (segment (start 131.953 78.613) (end 131.031099 79.534901) (width 0.25) (layer F.Cu) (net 8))
 (segment (start 131.953 72.4408) (end 131.953 78.613) (width 0.25) (layer F.Cu) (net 8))
 (segment (start 131.953 72.4408) (end 130.2639 70.7517) (width 0.25) (layer F.Cu) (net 8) (status 20))
 (segment (start 122.6439 63.1317) (end 122.1867 63.1317) (width 0.25) (layer F.Cu) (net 9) (status 30))
 (segment (start 122.1867 63.1317) (end 121.158 62.103) (width 0.25) (layer F.Cu) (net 9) (status 10))
 (segment (start 121.158 62.103) (end 117.549 62.103) (width 0.25) (layer F.Cu) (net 9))
 (segment (start 117.549 62.103) (end 117.227 62.425) (width 0.25) (layer F.Cu) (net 9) (status 20))
 (segment (start 122.6439 65.6717) (end 121.458507 65.6717) (width 0.25) (layer F.Cu) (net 10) (status 10))
 (segment (start 121.458507 65.6717) (end 120.855207 66.275) (width 0.25) (layer F.Cu) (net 10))
 (segment (start 120.855207 66.275) (end 118.677 66.275) (width 0.25) (layer F.Cu) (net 10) (status 20))
 (segment (start 122.1168 66.1988) (end 122.6439 65.6717) (width 0.25) (layer F.Cu) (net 10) (status 30))
 (segment (start 121.285 67.945) (end 121.215 67.875) (width 0.25) (layer F.Cu) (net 11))
 (segment (start 121.215 67.875) (end 118.677 67.875) (width 0.25) (layer F.Cu) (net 11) (status 20))
 (segment (start 121.285 69.3928) (end 121.285 67.945) (width 0.25) (layer F.Cu) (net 11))
 (segment (start 122.6439 70.7517) (end 121.285 69.3928) (width 0.25) (layer F.Cu) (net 11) (status 10))
 (segment (start 122.6439 70.7517) (end 122.4153 70.7517) (width 0.25) (layer F.Cu) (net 11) (status 30))
 (segment (start 112.427 70.925) (end 112.427 72.93) (width 0.25) (layer F.Cu) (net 12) (status 10))
 (segment (start 120.5357 78.3717) (end 122.6439 78.3717) (width 0.25) (layer F.Cu) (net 12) (status 20))
 (segment (start 116.713 74.549) (end 120.5357 78.3717) (width 0.25) (layer F.Cu) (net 12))
 (segment (start 114.046 74.549) (end 116.713 74.549) (width 0.25) (layer F.Cu) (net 12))
 (segment (start 112.427 72.93) (end 114.046 74.549) (width 0.25) (layer F.Cu) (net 12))
 (segment (start 122.1486 78.867) (end 122.6439 78.3717) (width 0.25) (layer F.Cu) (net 12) (status 30))
 (segment (start 113.227 72.841) (end 114.3 73.914) (width 0.25) (layer F.Cu) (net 13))
 (segment (start 113.227 70.925) (end 113.227 72.841) (width 0.25) (layer F.Cu) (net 13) (status 10))
 (segment (start 120.015 76.835) (end 123.317 76.835) (width 0.25) (layer F.Cu) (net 13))
 (segment (start 117.094 73.914) (end 120.015 76.835) (width 0.25) (layer F.Cu) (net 13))
 (segment (start 114.3 73.914) (end 117.094 73.914) (width 0.25) (layer F.Cu) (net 13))
 (segment (start 123.317 76.835) (end 124.8537 78.3717) (width 0.25) (layer F.Cu) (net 13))
 (segment (start 124.8537 78.3717) (end 130.2639 78.3717) (width 0.25) (layer F.Cu) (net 13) (status 20))
 (segment (start 114.027 70.925) (end 114.027 72.625) (width 0.25) (layer F.Cu) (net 14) (status 10))
 (segment (start 126.3523 75.8317) (end 125.857 76.327) (width 0.25) (layer F.Cu) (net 14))
 (segment (start 125.857 76.327) (end 120.523 76.327) (width 0.25) (layer F.Cu) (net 14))
 (segment (start 120.523 76.327) (end 117.475 73.279) (width 0.25) (layer F.Cu) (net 14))
 (segment (start 117.475 73.279) (end 114.681 73.279) (width 0.25) (layer F.Cu) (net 14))
 (segment (start 126.3523 75.8317) (end 130.2639 75.8317) (width 0.25) (layer F.Cu) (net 14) (status 20))
 (segment (start 114.027 72.625) (end 114.681 73.279) (width 0.25) (layer F.Cu) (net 14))
 (segment (start 113.919 71.033) (end 114.027 70.925) (width 0.25) (layer F.Cu) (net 14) (status 30))
 (segment (start 129.7686 76.327) (end 130.2639 75.8317) (width 0.25) (layer F.Cu) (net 14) (status 30))
 (segment (start 110.177 70) (end 110.177 69.475) (width 0.25) (layer F.Cu) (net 15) (status 20))
 (segment (start 109.093 71.084) (end 110.177 70) (width 0.25) (layer F.Cu) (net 15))
 (segment (start 109.093 79.121) (end 109.093 71.084) (width 0.25) (layer F.Cu) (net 15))
 (segment (start 110.109 80.137) (end 109.093 79.121) (width 0.25) (layer F.Cu) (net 15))
 (segment (start 131.319411 80.137) (end 110.109 80.137) (width 0.25) (layer F.Cu) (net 15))
 (segment (start 132.461 78.995411) (end 131.319411 80.137) (width 0.25) (layer F.Cu) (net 15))
 (segment (start 132.461 70.4088) (end 132.461 78.995411) (width 0.25) (layer F.Cu) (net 15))
 (segment (start 130.2639 68.2117) (end 132.461 70.4088) (width 0.25) (layer F.Cu) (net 15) (status 10))
 (segment (start 131.699 80.645) (end 133.223 79.121) (width 0.25) (layer F.Cu) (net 16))
 (segment (start 133.223 68.6308) (end 130.2639 65.6717) (width 0.25) (layer F.Cu) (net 16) (status 20))
 (segment (start 133.223 79.121) (end 133.223 68.6308) (width 0.25) (layer F.Cu) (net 16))
 (segment (start 131.699 80.645) (end 109.855 80.645) (width 0.25) (layer F.Cu) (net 16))
 (segment (start 108.585 79.375) (end 108.585 69.217) (width 0.25) (layer F.Cu) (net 16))
 (segment (start 109.855 80.645) (end 108.585 79.375) (width 0.25) (layer F.Cu) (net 16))
 (segment (start 109.127 68.675) (end 110.177 68.675) (width 0.25) (layer F.Cu) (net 16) (status 20))
 (segment (start 108.585 69.217) (end 109.127 68.675) (width 0.25) (layer F.Cu) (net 16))
 (segment (start 130.2639 65.6717) (end 130.2004 65.6717) (width 0.25) (layer B.Cu) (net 16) (status 30))
 (segment (start 130.2639 63.1317) (end 129.7813 63.1317) (width 0.25) (layer F.Cu) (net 17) (status 30))
 (segment (start 129.7813 63.1317) (end 128.524 64.389) (width 0.25) (layer F.Cu) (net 17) (status 10))
 (segment (start 120.65 65.532) (end 118.734 65.532) (width 0.25) (layer F.Cu) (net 17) (status 20))
 (segment (start 121.793 64.389) (end 120.65 65.532) (width 0.25) (layer F.Cu) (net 17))
 (segment (start 128.524 64.389) (end 121.793 64.389) (width 0.25) (layer F.Cu) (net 17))
 (segment (start 118.734 65.532) (end 118.677 65.475) (width 0.25) (layer F.Cu) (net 17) (status 30))
 (segment (start 130.1369 63.1317) (end 130.2639 63.1317) (width 0.25) (layer F.Cu) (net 17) (status 30))
 (segment (start 116.4224 70.8406) (end 116.4142 70.8488) (width 0.25) (layer F.Cu) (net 23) (status 30))
 (segment (start 139.446 67.818) (end 135.382 67.818) (width 0.25) (layer F.Cu) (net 18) (status 10))
 (segment (start 135.382 67.818) (end 134.366 68.834) (width 0.25) (layer F.Cu) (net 18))
 (segment (start 116.225 66.294) (end 116.225 70.886) (width 0.25) (layer B.Cu) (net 18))
 (segment (start 134.366 73.406) (end 134.366 68.834) (width 0.25) (layer F.Cu) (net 18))
 (via (at 134.366 73.406) (size 0.6) (drill 0.4) (layers F.Cu B.Cu) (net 18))
 (segment (start 133.223 74.549) (end 134.366 73.406) (width 0.25) (layer B.Cu) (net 18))
 (segment (start 128.143 74.549) (end 133.223 74.549) (width 0.25) (layer B.Cu) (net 18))
 (segment (start 127.127 75.565) (end 128.143 74.549) (width 0.25) (layer B.Cu) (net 18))
 (segment (start 120.904 75.565) (end 127.127 75.565) (width 0.25) (layer B.Cu) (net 18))
 (segment (start 116.225 70.886) (end 120.904 75.565) (width 0.25) (layer B.Cu) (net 18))
 (segment (start 116.225 66.401) (end 116.225 66.294) (width 0.25) (layer B.Cu) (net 18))
 (segment (start 116.225 66.294) (end 116.225 62.611) (width 0.25) (layer B.Cu) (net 18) (status 20))
 (segment (start 113.411 67.945) (end 114.681 67.945) (width 0.25) (layer B.Cu) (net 18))
 (segment (start 113.341 67.875) (end 113.411 67.945) (width 0.25) (layer F.Cu) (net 18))
 (via (at 113.411 67.945) (size 0.6) (drill 0.4) (layers F.Cu B.Cu) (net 18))
 (segment (start 110.177 67.875) (end 113.341 67.875) (width 0.25) (layer F.Cu) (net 18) (status 10))
 (segment (start 114.681 67.945) (end 116.225 66.401) (width 0.25) (layer B.Cu) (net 18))
 (segment (start 116.205 62.631) (end 116.225 62.611) (width 0.25) (layer B.Cu) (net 18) (status 30)))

